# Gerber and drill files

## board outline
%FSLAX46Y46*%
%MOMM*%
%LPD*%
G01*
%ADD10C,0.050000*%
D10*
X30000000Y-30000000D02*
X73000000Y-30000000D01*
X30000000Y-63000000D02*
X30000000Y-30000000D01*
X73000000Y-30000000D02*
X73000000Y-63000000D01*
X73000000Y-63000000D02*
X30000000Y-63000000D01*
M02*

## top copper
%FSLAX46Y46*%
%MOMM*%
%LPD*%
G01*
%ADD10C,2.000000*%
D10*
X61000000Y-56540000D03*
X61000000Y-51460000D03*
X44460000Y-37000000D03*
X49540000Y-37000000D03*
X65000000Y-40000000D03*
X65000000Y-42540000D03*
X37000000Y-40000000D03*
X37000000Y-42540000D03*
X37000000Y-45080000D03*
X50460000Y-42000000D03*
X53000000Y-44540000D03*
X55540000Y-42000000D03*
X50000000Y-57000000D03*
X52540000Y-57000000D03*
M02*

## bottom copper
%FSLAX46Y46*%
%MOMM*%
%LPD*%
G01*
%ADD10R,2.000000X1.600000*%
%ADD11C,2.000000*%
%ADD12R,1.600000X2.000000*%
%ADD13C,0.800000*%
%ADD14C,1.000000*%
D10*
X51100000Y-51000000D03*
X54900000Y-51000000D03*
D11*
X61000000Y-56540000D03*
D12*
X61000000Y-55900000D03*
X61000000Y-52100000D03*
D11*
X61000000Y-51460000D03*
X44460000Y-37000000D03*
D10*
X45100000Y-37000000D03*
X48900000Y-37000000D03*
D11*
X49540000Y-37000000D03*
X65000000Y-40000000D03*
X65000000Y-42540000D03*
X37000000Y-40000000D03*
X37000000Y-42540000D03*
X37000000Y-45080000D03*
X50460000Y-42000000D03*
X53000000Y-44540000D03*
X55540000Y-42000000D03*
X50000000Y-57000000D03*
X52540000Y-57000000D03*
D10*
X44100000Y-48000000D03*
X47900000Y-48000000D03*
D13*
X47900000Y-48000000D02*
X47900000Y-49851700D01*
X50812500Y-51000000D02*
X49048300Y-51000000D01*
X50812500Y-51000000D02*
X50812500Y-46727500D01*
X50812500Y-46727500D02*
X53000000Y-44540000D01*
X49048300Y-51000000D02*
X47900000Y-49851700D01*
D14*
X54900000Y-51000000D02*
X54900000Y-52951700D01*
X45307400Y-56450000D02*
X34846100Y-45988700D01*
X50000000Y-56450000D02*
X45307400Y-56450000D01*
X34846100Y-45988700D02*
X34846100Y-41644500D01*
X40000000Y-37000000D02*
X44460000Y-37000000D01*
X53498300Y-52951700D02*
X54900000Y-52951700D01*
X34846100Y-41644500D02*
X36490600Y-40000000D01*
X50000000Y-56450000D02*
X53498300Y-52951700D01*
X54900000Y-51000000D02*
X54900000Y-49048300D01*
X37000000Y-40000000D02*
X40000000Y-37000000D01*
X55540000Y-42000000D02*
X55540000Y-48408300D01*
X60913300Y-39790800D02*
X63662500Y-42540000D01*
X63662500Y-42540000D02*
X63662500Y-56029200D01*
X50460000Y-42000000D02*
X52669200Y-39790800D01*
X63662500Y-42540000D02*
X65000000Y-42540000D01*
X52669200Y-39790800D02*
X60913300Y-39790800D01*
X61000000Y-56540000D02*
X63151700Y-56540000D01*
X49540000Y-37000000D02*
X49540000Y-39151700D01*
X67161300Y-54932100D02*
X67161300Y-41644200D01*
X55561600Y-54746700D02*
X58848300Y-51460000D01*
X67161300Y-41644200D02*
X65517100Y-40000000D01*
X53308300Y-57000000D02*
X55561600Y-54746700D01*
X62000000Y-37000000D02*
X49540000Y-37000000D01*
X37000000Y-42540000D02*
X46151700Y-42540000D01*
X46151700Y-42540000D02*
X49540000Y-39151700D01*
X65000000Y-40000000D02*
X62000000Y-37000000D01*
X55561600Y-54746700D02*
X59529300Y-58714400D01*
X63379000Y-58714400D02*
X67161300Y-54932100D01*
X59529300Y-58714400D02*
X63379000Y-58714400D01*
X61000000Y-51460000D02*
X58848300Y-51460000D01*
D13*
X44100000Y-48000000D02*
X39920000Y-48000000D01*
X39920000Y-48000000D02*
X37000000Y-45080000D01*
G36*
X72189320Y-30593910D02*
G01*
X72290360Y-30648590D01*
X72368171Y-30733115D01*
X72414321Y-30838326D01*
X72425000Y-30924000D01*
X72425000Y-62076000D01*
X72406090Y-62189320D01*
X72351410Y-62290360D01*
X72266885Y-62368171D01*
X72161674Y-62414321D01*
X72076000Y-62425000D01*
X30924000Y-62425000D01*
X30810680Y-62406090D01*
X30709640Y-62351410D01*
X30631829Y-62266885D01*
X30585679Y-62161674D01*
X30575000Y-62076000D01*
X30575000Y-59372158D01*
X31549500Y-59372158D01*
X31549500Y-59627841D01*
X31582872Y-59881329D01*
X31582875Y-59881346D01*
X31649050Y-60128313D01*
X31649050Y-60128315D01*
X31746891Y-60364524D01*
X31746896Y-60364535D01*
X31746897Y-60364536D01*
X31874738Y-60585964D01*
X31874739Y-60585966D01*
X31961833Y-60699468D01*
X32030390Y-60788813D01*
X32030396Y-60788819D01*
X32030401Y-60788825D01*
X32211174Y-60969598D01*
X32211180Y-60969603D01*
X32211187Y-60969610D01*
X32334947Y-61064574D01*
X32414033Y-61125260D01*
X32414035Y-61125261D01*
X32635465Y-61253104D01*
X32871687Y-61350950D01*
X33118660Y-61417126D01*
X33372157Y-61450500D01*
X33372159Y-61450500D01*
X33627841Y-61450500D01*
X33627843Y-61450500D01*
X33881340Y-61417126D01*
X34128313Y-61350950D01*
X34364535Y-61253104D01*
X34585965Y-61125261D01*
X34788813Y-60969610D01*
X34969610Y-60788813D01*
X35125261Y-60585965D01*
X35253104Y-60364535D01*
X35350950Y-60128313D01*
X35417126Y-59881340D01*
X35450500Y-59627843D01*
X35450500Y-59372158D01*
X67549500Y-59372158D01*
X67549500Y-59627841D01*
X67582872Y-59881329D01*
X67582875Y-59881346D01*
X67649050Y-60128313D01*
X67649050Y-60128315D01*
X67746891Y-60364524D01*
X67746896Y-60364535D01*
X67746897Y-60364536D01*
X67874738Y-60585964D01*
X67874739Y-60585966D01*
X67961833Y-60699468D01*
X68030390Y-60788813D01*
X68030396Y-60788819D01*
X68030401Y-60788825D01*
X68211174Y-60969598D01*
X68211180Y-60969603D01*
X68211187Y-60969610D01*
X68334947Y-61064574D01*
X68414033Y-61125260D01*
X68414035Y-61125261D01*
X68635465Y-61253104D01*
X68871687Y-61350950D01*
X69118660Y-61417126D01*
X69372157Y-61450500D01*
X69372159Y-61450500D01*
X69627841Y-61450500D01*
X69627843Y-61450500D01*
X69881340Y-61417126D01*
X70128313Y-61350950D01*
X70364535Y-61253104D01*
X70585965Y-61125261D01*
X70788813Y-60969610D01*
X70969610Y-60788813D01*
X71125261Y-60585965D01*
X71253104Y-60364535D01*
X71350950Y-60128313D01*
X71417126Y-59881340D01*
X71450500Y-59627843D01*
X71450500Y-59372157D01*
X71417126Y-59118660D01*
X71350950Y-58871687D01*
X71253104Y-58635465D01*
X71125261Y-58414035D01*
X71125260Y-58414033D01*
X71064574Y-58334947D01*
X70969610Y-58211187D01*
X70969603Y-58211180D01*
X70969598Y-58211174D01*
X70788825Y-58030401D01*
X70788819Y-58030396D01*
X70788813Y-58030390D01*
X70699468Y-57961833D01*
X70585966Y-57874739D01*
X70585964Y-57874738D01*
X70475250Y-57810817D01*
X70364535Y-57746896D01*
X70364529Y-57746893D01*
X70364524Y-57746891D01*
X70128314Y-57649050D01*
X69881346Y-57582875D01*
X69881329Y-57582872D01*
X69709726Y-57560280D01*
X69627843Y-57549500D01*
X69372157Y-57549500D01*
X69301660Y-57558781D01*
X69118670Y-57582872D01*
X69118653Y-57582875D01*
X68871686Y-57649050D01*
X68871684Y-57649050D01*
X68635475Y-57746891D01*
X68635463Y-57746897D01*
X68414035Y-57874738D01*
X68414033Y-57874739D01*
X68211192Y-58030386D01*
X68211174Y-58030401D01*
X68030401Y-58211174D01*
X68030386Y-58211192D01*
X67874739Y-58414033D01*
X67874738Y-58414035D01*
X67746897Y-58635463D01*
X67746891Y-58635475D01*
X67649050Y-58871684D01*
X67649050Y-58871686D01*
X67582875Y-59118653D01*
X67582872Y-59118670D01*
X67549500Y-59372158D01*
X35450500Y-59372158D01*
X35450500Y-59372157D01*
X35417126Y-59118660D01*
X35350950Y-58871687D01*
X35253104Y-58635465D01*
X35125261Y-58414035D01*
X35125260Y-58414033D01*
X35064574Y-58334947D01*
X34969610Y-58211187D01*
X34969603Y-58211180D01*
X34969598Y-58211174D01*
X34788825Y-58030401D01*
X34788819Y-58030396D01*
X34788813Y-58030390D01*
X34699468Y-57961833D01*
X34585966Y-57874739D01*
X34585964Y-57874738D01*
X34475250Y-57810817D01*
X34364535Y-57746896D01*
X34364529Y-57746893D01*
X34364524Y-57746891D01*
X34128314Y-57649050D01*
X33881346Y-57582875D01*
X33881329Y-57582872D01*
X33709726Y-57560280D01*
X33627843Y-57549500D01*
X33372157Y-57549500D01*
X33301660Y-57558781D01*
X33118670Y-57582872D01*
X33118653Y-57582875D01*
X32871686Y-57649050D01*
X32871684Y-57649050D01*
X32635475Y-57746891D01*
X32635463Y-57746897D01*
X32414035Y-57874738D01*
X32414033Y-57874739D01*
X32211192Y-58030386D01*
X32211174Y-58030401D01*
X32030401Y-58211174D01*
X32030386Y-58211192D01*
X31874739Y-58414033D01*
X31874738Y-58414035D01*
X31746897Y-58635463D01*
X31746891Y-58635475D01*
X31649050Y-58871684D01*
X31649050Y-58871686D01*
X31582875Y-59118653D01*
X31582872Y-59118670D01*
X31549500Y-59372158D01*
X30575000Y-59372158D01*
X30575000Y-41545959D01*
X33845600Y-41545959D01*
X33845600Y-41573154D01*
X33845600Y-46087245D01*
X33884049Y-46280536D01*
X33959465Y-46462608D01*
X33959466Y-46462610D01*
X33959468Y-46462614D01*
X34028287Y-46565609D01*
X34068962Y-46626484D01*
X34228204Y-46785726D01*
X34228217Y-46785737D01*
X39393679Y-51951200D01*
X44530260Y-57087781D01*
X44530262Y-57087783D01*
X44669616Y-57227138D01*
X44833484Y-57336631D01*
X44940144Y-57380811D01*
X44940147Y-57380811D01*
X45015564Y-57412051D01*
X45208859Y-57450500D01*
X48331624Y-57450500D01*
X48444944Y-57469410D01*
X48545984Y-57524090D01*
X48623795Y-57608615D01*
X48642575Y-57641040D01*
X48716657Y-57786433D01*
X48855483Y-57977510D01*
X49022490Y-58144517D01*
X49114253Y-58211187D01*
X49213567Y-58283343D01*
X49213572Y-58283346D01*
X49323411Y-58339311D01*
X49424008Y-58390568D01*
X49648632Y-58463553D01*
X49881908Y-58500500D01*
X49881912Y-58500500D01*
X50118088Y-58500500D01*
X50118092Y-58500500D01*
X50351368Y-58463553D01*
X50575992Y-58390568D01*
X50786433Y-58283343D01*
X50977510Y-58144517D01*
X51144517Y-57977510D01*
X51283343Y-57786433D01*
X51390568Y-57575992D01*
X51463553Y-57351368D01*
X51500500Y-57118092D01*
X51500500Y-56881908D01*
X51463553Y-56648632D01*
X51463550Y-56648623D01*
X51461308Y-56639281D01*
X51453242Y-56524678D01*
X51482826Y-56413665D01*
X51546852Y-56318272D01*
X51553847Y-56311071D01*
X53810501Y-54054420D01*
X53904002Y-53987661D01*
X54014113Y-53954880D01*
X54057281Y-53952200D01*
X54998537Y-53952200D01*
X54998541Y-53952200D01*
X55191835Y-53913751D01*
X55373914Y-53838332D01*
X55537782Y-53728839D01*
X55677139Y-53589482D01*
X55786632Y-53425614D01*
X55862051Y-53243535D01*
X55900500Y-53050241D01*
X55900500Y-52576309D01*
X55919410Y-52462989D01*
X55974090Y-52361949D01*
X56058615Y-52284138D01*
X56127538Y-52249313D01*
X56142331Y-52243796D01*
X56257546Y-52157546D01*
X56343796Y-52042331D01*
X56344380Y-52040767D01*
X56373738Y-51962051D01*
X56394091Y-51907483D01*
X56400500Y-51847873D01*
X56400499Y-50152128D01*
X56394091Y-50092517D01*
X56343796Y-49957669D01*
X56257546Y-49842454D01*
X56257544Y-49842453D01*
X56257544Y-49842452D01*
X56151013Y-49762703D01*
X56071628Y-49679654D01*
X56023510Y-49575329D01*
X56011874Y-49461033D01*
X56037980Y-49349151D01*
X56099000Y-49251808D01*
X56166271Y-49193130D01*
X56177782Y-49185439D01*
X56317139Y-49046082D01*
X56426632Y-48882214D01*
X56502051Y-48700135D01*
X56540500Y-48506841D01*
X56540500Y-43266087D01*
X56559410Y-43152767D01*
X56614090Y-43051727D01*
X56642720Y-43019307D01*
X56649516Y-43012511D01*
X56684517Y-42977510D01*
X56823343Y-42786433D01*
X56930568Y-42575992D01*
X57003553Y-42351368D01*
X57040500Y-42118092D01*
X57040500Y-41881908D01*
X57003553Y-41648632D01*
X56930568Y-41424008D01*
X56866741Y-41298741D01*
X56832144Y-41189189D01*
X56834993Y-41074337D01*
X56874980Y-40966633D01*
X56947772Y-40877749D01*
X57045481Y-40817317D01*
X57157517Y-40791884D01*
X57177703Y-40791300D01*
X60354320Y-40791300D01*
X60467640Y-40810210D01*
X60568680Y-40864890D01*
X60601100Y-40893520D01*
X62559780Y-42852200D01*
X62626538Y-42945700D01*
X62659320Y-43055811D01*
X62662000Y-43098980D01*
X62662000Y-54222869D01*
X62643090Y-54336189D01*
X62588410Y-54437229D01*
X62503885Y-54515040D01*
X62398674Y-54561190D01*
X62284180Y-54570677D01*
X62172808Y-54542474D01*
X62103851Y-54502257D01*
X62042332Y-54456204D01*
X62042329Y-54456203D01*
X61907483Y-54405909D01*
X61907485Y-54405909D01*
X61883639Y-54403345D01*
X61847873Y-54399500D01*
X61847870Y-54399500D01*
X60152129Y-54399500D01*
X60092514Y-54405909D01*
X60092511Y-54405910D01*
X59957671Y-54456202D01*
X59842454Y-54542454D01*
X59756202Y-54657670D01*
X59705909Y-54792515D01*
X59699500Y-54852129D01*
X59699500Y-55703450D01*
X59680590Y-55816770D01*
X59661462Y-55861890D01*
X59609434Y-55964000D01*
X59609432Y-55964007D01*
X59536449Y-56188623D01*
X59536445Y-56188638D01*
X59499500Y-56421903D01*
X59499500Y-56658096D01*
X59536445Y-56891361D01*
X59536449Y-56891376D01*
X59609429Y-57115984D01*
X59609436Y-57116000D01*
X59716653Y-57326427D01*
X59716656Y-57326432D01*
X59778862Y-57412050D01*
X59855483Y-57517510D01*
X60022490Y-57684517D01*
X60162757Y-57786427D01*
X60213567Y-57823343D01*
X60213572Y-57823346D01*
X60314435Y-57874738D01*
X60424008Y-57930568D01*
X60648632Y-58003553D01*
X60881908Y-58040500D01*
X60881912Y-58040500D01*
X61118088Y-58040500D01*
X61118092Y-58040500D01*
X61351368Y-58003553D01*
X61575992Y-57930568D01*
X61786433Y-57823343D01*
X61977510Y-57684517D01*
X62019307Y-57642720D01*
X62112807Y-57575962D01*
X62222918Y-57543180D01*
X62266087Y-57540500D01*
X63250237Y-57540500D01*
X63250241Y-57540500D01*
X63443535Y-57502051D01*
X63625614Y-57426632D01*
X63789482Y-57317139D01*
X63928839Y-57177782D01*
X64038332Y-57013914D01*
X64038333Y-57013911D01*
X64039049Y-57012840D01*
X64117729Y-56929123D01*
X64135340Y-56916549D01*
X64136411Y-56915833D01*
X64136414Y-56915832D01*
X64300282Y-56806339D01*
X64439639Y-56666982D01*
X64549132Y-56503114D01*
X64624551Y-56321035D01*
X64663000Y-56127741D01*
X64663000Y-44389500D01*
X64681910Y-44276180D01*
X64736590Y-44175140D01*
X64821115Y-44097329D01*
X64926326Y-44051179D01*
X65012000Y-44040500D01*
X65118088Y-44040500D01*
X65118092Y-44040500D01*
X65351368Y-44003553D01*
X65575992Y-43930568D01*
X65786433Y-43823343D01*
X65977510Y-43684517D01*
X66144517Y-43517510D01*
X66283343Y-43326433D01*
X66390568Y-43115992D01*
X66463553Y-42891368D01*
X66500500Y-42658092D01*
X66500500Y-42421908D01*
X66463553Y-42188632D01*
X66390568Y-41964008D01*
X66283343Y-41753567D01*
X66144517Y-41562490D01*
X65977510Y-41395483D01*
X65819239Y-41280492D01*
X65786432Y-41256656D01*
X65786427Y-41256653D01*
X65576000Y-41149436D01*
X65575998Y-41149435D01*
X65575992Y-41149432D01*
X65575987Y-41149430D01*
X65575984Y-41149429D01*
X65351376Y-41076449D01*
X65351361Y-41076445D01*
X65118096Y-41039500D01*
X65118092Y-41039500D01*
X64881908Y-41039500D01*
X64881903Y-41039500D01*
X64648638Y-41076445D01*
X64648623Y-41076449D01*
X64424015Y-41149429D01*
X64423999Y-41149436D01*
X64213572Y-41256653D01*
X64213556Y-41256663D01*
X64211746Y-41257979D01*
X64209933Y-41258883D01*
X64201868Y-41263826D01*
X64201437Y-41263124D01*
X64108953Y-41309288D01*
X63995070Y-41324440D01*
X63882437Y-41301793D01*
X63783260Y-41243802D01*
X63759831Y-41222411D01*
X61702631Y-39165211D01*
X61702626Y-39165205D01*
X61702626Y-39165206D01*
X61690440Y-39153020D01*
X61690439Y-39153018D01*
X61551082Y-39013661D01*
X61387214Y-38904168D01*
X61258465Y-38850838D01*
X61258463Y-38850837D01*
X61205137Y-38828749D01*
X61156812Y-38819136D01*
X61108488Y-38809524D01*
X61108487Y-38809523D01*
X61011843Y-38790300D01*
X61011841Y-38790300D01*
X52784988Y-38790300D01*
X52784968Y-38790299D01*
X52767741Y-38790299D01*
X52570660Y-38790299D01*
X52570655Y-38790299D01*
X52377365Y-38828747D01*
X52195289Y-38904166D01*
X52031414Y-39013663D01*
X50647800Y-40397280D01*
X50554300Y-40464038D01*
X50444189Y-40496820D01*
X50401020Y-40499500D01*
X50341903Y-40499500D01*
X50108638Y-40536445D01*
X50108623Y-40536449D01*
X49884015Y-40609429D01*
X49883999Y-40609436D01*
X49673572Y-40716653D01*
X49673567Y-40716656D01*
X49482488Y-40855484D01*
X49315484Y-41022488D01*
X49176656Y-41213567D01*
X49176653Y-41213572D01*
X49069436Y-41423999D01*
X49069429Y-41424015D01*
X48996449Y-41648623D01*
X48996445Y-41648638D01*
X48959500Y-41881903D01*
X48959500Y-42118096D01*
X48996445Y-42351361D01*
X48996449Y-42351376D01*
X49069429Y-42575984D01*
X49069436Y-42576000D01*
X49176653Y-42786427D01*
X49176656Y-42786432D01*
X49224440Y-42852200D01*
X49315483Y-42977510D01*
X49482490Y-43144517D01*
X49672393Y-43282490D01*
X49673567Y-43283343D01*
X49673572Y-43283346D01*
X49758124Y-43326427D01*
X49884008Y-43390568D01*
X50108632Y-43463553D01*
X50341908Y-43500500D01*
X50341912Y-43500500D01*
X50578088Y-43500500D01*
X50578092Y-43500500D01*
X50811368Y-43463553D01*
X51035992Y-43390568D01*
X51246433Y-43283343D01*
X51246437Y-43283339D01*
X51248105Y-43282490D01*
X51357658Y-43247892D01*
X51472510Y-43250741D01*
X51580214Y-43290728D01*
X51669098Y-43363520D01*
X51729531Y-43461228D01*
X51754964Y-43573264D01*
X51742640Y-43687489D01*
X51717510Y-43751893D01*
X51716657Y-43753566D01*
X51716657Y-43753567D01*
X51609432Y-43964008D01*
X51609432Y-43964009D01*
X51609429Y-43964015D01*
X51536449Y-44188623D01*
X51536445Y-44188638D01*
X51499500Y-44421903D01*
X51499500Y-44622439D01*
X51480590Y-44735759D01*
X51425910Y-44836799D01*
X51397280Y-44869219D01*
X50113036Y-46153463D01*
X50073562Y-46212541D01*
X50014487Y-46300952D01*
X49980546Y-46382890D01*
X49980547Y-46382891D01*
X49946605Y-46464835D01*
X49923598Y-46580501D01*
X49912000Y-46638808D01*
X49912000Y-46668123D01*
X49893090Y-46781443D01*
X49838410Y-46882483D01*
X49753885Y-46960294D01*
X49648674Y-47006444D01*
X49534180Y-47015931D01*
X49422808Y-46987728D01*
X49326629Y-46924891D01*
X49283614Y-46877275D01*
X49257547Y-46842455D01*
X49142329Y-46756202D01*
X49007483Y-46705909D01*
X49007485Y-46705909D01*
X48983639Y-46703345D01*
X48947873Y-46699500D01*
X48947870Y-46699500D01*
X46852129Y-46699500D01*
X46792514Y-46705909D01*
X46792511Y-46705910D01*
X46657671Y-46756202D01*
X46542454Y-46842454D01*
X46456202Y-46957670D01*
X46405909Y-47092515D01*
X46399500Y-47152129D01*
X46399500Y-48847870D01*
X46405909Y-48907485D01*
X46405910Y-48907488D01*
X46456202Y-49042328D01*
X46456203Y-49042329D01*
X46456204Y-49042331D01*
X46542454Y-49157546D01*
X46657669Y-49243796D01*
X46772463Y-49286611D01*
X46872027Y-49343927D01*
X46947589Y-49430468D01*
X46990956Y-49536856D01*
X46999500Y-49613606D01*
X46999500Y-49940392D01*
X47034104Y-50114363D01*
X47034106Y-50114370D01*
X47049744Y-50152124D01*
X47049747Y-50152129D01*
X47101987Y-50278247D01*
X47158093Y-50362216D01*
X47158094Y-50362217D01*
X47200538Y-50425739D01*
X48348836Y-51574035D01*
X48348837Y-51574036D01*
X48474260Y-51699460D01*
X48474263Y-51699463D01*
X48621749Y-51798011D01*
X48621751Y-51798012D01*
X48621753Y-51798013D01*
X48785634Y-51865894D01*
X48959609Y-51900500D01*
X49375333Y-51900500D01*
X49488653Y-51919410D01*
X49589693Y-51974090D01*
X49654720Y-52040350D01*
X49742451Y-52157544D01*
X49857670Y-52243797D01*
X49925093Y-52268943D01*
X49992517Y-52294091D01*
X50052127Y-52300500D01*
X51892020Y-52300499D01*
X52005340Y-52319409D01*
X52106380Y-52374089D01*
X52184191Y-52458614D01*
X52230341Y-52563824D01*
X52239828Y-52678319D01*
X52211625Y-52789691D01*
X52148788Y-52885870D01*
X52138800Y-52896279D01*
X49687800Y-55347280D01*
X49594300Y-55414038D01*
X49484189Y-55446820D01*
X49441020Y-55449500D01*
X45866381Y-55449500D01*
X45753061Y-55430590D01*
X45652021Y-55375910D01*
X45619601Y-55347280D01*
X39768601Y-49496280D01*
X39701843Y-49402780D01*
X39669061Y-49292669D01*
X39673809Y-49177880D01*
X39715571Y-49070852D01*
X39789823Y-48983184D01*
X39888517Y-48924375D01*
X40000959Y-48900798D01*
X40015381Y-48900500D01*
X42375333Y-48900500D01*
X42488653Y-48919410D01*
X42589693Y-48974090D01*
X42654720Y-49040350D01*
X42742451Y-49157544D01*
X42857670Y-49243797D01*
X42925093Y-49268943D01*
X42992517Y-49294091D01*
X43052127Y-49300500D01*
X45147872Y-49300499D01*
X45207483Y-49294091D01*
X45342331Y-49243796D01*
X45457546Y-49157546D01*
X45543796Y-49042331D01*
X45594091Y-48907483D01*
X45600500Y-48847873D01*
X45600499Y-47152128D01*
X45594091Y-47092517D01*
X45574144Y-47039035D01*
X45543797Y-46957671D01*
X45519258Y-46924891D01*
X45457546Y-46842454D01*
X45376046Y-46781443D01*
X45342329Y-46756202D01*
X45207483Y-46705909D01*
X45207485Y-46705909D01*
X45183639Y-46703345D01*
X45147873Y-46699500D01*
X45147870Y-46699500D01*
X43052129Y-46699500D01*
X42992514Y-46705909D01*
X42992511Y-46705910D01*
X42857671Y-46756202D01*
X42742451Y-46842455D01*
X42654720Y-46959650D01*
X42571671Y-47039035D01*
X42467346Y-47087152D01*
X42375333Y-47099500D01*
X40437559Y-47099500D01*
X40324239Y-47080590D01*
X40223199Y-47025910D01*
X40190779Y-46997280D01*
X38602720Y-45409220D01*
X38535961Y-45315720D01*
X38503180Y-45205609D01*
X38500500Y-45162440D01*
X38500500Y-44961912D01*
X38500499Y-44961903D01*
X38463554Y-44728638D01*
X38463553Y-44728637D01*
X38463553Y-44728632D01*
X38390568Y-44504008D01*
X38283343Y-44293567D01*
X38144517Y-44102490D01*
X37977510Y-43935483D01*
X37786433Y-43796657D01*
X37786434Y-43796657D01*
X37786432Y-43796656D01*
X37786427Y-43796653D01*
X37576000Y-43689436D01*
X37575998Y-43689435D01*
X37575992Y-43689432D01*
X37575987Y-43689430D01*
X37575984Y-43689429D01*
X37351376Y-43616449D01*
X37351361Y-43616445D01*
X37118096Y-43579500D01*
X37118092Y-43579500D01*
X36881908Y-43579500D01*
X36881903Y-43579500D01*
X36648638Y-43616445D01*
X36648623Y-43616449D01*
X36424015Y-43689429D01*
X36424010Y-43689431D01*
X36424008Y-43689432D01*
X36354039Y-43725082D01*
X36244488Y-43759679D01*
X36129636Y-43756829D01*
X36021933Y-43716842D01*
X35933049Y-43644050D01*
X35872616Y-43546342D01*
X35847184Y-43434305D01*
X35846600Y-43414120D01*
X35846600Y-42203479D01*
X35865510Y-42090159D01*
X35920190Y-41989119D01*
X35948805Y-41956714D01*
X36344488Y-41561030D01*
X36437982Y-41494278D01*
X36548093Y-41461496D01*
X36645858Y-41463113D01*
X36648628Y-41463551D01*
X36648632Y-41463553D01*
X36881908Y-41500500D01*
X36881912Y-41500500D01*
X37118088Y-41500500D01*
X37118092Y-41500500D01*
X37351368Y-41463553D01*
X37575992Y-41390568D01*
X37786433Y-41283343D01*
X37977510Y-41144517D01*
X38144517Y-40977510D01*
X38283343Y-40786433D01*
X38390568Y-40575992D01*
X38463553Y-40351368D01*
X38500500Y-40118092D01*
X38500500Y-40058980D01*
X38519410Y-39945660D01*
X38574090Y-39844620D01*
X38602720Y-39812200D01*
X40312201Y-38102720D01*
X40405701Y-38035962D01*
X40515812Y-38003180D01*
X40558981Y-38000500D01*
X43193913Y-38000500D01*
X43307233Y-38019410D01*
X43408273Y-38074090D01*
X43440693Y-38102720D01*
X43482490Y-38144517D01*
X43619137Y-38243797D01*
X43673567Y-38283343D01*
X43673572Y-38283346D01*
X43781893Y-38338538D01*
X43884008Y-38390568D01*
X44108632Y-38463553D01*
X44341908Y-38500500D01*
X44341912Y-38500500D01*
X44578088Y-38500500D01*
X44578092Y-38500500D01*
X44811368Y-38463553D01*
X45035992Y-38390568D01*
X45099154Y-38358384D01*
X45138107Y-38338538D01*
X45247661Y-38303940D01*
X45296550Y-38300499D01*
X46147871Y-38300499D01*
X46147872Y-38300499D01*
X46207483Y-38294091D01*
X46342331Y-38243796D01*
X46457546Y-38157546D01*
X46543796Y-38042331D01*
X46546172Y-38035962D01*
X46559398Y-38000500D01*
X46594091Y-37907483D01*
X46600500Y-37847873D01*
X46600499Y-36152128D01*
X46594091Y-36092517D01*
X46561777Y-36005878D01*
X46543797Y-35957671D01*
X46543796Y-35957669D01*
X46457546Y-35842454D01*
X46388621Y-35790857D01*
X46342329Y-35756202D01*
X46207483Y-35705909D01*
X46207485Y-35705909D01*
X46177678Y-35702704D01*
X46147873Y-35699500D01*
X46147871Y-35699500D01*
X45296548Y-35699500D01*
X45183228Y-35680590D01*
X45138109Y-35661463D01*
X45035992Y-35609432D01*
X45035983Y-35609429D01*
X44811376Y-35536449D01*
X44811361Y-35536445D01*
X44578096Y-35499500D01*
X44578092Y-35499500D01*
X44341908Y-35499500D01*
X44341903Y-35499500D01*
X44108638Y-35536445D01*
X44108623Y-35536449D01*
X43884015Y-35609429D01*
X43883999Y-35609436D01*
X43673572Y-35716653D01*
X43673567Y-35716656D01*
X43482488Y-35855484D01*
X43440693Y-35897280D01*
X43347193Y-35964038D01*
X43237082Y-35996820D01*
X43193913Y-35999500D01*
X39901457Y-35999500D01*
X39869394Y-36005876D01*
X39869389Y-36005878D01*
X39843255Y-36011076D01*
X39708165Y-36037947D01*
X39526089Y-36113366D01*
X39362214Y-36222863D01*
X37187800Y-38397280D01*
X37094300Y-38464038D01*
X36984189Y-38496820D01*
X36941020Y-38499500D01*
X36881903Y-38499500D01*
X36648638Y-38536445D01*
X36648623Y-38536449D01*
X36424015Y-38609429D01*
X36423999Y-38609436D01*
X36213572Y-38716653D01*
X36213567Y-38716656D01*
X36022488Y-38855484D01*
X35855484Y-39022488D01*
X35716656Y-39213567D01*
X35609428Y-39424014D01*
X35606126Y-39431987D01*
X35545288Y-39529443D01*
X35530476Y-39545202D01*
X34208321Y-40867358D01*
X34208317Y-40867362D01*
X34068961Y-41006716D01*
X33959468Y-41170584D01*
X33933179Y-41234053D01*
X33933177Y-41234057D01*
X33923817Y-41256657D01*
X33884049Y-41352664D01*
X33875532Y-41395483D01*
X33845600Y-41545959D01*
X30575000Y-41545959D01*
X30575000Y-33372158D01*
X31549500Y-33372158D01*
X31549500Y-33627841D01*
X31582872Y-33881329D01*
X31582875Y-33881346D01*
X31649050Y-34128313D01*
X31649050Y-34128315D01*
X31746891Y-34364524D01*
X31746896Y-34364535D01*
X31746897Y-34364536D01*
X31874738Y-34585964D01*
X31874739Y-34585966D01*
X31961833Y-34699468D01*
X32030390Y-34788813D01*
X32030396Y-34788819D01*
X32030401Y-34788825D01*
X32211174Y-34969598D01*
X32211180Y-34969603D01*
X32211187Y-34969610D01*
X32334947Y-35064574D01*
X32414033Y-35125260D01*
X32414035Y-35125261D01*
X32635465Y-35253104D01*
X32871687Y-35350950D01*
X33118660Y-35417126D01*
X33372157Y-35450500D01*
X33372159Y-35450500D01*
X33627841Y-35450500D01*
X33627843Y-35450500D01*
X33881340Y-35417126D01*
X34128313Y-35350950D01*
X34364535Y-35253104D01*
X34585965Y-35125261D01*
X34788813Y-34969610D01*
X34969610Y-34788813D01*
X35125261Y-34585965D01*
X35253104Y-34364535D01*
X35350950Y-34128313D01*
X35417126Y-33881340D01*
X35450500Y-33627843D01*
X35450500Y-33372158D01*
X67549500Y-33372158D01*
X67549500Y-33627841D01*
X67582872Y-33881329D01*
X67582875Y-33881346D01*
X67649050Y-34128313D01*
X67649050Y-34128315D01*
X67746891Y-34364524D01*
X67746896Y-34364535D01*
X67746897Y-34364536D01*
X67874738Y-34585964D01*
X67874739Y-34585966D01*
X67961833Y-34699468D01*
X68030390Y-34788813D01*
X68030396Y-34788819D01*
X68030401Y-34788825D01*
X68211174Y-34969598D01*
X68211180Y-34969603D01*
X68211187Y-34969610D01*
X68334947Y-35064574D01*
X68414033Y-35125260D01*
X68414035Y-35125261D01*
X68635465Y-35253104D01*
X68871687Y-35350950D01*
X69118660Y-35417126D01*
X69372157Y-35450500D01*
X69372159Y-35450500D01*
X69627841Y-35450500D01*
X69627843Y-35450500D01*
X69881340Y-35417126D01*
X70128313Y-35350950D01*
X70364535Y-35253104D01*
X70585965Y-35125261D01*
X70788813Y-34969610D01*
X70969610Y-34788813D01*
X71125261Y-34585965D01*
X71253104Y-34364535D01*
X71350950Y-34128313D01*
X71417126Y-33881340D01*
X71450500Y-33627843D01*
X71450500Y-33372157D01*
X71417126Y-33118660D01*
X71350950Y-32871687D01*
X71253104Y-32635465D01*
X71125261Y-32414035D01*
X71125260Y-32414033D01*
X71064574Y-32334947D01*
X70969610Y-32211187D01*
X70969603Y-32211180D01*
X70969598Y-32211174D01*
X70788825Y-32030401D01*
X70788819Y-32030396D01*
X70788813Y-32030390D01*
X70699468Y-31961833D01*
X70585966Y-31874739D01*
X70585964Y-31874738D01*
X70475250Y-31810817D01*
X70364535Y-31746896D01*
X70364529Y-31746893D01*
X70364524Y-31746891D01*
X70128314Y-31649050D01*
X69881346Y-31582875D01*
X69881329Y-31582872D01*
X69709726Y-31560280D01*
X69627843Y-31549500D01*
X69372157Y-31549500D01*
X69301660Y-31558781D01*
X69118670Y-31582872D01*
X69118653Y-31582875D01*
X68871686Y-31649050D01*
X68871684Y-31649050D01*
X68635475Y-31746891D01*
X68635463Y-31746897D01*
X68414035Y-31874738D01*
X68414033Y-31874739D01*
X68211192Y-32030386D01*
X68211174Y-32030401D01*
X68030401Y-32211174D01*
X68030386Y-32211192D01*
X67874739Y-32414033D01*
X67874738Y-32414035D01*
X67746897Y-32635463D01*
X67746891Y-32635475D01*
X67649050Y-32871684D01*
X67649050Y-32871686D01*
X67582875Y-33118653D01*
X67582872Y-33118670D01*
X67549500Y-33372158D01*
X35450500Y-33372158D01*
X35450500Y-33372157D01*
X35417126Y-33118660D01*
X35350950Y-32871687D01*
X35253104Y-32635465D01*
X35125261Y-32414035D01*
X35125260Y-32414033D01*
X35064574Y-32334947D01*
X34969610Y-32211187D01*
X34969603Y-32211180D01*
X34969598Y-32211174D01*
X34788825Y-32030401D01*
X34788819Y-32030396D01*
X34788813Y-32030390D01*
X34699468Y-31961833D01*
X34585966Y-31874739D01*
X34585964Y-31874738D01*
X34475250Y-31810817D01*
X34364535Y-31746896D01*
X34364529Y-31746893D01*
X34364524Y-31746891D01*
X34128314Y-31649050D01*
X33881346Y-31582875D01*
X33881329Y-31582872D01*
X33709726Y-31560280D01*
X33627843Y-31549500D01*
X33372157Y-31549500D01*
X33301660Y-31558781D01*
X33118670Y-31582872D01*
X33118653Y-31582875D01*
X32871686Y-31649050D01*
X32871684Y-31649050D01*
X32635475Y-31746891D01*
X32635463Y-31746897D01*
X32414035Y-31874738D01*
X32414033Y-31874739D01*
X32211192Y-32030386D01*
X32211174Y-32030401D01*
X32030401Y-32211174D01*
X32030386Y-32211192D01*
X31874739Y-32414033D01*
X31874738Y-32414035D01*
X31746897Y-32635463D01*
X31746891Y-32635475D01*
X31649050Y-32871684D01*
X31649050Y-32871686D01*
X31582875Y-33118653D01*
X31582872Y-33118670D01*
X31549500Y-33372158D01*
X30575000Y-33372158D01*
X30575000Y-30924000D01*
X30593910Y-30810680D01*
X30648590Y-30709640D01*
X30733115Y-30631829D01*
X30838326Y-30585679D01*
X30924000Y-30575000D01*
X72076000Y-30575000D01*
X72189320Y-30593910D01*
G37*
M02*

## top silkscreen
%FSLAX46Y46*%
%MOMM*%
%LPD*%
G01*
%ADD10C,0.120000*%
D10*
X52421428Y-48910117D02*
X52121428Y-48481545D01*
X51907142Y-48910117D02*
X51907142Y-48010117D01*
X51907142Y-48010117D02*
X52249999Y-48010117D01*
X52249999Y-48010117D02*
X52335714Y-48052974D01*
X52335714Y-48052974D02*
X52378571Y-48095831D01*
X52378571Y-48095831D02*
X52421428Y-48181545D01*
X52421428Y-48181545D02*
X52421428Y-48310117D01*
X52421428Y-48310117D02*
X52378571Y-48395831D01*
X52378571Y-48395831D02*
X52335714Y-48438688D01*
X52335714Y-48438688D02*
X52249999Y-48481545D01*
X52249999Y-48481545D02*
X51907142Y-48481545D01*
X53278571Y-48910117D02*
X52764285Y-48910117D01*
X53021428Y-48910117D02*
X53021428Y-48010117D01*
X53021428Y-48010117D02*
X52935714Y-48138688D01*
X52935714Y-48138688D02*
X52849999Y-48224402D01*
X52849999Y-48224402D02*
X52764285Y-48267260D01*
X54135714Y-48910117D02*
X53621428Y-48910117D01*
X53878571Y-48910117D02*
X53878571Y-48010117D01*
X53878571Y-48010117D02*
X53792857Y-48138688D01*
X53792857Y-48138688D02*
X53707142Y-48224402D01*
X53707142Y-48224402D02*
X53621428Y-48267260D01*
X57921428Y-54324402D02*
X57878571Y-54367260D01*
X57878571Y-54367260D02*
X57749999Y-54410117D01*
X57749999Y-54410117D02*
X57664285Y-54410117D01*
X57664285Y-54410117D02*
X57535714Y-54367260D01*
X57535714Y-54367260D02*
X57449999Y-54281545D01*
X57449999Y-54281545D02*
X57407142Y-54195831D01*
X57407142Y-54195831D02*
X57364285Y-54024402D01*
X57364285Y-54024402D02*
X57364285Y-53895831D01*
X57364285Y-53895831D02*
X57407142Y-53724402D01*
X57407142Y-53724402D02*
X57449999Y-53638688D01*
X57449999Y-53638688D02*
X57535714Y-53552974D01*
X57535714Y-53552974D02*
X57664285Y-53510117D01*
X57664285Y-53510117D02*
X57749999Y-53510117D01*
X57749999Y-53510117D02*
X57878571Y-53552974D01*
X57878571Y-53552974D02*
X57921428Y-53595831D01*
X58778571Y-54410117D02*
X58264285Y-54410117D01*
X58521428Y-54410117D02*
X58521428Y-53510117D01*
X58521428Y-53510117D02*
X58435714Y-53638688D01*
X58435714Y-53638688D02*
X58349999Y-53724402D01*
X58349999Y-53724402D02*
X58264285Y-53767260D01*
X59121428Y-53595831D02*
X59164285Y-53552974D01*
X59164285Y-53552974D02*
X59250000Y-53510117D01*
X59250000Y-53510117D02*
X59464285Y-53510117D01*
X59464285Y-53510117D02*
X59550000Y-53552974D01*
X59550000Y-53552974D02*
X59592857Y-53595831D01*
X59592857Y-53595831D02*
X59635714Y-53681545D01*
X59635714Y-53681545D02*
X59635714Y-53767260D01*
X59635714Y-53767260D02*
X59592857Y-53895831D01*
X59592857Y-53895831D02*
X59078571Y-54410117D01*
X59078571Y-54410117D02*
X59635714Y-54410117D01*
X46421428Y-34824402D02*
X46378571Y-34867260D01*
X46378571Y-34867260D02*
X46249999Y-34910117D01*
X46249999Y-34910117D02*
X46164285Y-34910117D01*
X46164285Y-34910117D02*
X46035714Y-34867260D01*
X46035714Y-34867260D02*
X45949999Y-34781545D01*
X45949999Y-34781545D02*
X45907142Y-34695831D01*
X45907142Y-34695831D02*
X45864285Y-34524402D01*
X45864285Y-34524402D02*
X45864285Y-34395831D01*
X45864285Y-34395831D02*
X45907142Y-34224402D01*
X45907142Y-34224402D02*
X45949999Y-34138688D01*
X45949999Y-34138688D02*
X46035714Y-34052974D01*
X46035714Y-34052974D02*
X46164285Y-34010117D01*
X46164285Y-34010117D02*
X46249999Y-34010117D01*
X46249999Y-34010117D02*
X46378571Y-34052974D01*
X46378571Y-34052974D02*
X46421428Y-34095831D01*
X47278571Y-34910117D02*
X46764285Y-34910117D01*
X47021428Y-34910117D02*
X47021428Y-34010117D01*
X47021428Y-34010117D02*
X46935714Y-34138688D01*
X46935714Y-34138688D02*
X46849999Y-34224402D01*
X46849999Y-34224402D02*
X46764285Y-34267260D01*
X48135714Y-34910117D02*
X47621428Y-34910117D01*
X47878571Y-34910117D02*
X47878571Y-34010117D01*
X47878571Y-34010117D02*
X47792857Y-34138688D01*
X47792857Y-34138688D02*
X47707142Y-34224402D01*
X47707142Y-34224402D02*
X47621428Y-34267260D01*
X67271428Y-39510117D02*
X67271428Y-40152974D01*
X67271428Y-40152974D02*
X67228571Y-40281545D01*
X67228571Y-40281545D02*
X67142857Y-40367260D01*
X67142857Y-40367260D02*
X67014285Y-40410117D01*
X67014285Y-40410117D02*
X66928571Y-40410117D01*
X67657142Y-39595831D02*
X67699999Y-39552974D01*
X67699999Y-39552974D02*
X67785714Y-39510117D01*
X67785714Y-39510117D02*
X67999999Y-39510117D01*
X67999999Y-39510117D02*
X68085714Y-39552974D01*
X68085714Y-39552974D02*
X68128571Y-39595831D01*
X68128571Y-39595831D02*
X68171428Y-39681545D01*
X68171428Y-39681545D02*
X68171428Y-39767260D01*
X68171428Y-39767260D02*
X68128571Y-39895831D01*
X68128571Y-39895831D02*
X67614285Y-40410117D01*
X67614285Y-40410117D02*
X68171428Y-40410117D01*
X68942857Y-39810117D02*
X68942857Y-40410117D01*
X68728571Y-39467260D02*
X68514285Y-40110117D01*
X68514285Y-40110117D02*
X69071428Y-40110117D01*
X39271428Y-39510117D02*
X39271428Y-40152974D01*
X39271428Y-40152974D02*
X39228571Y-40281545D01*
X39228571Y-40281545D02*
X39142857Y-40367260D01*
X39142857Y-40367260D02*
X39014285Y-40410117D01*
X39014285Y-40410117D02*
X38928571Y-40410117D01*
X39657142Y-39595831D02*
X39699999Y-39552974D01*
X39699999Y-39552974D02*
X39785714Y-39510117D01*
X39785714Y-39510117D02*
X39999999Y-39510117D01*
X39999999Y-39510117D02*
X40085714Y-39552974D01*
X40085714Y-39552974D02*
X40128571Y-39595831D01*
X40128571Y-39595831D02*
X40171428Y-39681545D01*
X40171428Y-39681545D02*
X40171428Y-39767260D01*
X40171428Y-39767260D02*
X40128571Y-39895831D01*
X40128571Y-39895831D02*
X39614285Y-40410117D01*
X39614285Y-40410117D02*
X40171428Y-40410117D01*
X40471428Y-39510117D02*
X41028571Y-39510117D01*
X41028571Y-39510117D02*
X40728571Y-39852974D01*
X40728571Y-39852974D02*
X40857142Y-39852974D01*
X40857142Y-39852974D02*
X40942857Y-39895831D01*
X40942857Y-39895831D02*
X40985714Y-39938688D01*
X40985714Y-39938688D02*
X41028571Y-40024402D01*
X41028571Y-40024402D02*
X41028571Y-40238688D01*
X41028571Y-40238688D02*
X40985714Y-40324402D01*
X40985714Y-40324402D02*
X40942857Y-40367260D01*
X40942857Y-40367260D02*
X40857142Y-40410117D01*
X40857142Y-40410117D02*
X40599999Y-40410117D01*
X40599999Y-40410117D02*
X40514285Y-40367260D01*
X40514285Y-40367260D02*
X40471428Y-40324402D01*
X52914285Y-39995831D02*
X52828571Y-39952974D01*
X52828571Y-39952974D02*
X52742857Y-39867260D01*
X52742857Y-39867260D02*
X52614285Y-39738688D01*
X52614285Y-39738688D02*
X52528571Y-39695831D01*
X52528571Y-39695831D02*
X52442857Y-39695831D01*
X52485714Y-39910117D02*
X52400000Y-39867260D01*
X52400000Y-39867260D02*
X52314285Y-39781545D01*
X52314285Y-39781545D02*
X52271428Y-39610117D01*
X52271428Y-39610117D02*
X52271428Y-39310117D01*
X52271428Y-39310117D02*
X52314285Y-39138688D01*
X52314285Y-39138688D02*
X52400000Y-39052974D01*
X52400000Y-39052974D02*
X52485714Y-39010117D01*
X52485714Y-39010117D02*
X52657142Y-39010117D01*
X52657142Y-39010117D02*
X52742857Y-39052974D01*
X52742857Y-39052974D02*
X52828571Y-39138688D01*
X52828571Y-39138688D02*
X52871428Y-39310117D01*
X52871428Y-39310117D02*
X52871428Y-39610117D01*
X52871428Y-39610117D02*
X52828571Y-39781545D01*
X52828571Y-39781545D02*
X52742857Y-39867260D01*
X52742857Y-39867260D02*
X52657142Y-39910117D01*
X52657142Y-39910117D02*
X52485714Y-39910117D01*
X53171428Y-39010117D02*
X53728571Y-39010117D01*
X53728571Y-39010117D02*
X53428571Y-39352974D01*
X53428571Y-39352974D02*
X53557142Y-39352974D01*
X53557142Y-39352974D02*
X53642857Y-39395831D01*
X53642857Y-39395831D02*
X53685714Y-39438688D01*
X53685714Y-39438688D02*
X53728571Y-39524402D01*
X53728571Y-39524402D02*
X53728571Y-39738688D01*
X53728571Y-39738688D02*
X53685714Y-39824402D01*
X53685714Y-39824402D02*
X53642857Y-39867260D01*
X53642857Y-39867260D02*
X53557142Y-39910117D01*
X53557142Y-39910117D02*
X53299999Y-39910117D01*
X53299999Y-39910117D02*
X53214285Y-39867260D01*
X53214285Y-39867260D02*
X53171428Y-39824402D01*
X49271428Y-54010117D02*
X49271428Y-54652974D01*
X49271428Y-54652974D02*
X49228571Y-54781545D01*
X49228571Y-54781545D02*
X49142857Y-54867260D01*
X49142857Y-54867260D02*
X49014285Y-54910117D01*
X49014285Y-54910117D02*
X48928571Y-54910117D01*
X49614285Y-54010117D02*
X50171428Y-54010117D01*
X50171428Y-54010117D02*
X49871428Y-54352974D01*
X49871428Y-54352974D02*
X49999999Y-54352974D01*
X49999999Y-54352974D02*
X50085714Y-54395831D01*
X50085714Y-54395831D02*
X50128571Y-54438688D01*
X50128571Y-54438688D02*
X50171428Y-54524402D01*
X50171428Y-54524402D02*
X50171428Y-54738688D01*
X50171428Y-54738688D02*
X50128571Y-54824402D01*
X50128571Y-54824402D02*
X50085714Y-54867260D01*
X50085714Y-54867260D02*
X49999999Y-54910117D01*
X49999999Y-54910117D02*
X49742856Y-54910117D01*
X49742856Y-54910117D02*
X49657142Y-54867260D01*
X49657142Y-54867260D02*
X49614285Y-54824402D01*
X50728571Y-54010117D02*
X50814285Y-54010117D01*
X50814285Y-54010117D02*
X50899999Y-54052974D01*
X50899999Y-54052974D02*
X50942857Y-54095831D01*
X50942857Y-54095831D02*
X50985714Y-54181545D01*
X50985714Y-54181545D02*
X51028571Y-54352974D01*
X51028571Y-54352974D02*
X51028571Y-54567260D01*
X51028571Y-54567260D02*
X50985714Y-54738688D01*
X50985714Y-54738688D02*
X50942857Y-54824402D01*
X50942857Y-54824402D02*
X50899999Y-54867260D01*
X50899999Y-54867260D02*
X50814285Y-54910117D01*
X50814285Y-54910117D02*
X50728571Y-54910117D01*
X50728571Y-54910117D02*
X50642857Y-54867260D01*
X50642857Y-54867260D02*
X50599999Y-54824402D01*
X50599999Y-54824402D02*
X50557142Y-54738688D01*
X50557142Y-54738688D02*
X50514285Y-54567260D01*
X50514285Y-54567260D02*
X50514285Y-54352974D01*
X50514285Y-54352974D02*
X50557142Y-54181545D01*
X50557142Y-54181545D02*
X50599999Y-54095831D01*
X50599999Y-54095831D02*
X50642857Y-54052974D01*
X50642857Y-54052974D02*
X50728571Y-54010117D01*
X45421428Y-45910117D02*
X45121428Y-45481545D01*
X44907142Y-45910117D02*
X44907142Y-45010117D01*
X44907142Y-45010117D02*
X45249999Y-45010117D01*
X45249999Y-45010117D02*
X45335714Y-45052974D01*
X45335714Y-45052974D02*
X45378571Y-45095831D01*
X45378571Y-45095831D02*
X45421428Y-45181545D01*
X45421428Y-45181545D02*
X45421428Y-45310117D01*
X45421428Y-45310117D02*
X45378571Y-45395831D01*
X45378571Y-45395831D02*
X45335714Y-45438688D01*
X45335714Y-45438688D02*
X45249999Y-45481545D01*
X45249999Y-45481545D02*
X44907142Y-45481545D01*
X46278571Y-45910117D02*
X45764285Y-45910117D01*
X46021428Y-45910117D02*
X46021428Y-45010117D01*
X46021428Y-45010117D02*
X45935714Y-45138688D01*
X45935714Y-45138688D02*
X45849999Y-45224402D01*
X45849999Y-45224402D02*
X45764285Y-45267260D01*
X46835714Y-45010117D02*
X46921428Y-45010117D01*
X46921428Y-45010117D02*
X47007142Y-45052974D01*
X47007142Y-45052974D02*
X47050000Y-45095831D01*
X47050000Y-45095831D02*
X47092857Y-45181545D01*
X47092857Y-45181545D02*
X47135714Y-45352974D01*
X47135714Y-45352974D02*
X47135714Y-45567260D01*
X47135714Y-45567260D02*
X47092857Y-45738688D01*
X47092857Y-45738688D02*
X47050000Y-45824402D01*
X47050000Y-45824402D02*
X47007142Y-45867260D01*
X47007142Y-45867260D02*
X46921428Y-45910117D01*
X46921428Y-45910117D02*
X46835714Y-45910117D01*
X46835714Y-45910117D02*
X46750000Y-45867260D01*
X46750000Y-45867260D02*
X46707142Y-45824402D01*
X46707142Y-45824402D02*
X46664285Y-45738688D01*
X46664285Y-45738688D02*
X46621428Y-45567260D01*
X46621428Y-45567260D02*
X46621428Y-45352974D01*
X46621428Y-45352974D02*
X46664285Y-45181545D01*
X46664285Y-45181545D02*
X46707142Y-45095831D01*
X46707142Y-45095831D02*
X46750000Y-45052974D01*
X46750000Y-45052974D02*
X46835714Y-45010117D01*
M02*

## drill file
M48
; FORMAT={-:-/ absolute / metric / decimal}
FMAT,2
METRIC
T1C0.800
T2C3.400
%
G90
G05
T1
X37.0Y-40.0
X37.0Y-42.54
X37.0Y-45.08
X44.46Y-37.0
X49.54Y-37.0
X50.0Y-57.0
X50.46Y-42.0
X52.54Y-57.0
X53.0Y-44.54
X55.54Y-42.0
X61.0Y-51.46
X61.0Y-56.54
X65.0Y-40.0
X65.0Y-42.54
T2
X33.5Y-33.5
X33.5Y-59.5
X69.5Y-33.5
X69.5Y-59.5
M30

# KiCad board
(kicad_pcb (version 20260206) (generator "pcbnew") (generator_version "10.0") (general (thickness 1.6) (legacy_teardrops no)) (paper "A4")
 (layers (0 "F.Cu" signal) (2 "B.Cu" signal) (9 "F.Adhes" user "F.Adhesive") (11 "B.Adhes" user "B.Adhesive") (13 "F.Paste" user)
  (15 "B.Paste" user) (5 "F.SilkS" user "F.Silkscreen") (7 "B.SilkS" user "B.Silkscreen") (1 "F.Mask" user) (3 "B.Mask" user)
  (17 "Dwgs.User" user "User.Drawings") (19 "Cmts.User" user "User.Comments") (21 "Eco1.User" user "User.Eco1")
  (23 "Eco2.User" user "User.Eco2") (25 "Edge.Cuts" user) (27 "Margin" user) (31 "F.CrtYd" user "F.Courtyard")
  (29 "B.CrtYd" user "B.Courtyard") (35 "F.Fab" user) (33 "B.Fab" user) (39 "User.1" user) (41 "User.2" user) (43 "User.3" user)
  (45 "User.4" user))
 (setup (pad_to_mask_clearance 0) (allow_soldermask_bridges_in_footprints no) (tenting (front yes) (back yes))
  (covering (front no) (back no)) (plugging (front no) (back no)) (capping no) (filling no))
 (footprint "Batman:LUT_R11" (layer "F.Cu") (at 53 51)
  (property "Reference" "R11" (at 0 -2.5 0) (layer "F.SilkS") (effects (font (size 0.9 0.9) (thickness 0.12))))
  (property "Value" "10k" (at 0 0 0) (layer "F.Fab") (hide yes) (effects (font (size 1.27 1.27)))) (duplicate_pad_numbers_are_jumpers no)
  (pad "1" smd rect (at -1.9 0) (size 2 1.6) (layers "B.Cu") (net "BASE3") (thermal_bridge_angle 45))
  (pad "2" smd rect (at 1.9 0) (size 2 1.6) (layers "B.Cu") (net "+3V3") (thermal_bridge_angle 45)))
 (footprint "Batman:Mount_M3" (layer "F.Cu") (at 69.5 33.5)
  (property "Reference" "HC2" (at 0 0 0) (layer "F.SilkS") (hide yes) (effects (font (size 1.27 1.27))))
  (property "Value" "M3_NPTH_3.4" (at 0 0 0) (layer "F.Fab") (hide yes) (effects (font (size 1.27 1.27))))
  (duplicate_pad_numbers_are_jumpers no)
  (pad "" np_thru_hole circle (at 0 0) (size 3.4 3.4) (drill 3.4) (layers "*.Cu")))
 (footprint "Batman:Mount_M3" (layer "F.Cu") (at 33.5 59.5)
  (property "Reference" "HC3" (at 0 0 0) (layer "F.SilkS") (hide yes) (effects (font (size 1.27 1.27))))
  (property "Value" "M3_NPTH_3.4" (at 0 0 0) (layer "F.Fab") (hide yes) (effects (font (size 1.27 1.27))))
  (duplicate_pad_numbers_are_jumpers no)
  (pad "" np_thru_hole circle (at 0 0) (size 3.4 3.4) (drill 3.4) (layers "*.Cu")))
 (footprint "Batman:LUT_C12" (layer "F.Cu") (at 61 54 90)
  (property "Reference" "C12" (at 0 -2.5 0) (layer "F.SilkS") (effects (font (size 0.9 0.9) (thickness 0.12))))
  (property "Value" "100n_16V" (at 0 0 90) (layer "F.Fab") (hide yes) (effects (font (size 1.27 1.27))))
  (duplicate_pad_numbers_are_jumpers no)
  (pad "1" thru_hole circle (at -2.54 0 90) (size 2 2) (drill 0.8) (layers "*.Cu") (remove_unused_layers no) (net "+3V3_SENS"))
  (pad "1" smd rect (at -1.9 0 90) (size 2 1.6) (layers "B.Cu") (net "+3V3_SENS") (thermal_bridge_angle 45))
  (pad "2" smd rect (at 1.9 0 90) (size 2 1.6) (layers "B.Cu") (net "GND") (thermal_bridge_angle 45))
  (pad "2" thru_hole circle (at 2.54 0 90) (size 2 2) (drill 0.8) (layers "*.Cu") (remove_unused_layers no) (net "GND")))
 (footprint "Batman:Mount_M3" (layer "F.Cu") (at 33.5 33.5)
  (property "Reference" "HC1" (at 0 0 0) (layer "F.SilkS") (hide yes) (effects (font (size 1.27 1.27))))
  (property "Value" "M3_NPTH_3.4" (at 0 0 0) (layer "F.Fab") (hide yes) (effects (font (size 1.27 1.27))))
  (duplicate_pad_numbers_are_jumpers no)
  (pad "" np_thru_hole circle (at 0 0) (size 3.4 3.4) (drill 3.4) (layers "*.Cu")))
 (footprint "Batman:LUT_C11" (layer "F.Cu") (at 47 37)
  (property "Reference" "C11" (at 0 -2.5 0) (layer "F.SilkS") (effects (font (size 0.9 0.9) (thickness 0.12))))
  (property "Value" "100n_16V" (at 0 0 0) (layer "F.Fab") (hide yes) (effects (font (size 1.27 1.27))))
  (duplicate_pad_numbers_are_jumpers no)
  (pad "1" thru_hole circle (at -2.54 0) (size 2 2) (drill 0.8) (layers "*.Cu") (remove_unused_layers no) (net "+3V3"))
  (pad "1" smd rect (at -1.9 0) (size 2 1.6) (layers "B.Cu") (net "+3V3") (thermal_bridge_angle 45))
  (pad "2" smd rect (at 1.9 0) (size 2 1.6) (layers "B.Cu") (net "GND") (thermal_bridge_angle 45))
  (pad "2" thru_hole circle (at 2.54 0) (size 2 2) (drill 0.8) (layers "*.Cu") (remove_unused_layers no) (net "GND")))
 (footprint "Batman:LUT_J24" (layer "F.Cu") (at 65 40 -90)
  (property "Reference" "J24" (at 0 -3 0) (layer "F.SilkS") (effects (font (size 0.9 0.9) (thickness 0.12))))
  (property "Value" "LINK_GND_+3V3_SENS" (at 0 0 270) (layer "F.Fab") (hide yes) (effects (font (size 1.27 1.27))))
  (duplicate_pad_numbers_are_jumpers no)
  (pad "1" thru_hole circle (at 0 0 270) (size 2 2) (drill 0.8) (layers "*.Cu") (remove_unused_layers no) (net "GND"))
  (pad "2" thru_hole circle (at 2.54 0 270) (size 2 2) (drill 0.8) (layers "*.Cu") (remove_unused_layers no) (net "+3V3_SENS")))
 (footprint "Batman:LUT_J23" (layer "F.Cu") (at 37 40 -90)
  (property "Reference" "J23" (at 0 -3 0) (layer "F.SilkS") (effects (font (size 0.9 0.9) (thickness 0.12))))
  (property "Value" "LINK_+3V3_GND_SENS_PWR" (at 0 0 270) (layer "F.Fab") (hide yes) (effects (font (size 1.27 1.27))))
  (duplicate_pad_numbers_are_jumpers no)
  (pad "1" thru_hole circle (at 0 0 270) (size 2 2) (drill 0.8) (layers "*.Cu") (remove_unused_layers no) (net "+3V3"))
  (pad "2" thru_hole circle (at 2.54 0 270) (size 2 2) (drill 0.8) (layers "*.Cu") (remove_unused_layers no) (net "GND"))
  (pad "3" thru_hole circle (at 5.08 0 270) (size 2 2) (drill 0.8) (layers "*.Cu") (remove_unused_layers no) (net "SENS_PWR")))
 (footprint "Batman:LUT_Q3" (layer "F.Cu") (at 53 42)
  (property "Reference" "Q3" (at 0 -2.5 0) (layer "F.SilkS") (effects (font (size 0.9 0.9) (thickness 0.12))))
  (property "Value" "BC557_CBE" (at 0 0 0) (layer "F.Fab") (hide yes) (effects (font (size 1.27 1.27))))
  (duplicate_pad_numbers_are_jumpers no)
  (pad "1" thru_hole circle (at -2.54 0) (size 2 2) (drill 0.8) (layers "*.Cu") (remove_unused_layers no) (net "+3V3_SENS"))
  (pad "2" thru_hole circle (at 0 2.54) (size 2 2) (drill 0.8) (layers "*.Cu") (remove_unused_layers no) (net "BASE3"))
  (pad "3" thru_hole circle (at 2.54 0) (size 2 2) (drill 0.8) (layers "*.Cu") (remove_unused_layers no) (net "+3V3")))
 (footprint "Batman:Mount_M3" (layer "F.Cu") (at 69.5 59.5)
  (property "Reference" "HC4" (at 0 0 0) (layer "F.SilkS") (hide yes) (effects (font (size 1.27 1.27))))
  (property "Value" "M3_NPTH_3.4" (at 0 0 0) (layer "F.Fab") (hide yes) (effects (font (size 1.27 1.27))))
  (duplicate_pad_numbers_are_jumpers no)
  (pad "" np_thru_hole circle (at 0 0) (size 3.4 3.4) (drill 3.4) (layers "*.Cu")))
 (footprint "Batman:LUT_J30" (layer "F.Cu") (at 50 57)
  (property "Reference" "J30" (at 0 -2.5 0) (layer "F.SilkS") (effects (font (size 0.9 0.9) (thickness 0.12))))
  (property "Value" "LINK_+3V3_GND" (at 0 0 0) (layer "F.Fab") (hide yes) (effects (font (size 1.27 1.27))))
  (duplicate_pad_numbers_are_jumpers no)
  (pad "1" thru_hole circle (at 0 0) (size 2 2) (drill 0.8) (layers "*.Cu") (remove_unused_layers no) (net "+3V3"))
  (pad "2" thru_hole circle (at 2.54 0) (size 2 2) (drill 0.8) (layers "*.Cu") (remove_unused_layers no) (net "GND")))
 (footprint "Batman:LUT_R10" (layer "F.Cu") (at 46 48)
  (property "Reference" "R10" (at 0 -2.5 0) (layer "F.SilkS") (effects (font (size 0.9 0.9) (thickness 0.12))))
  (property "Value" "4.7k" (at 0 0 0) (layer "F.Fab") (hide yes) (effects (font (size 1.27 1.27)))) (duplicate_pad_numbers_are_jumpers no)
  (pad "1" smd rect (at -1.9 0) (size 2 1.6) (layers "B.Cu") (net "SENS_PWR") (thermal_bridge_angle 45))
  (pad "2" smd rect (at 1.9 0) (size 2 1.6) (layers "B.Cu") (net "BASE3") (thermal_bridge_angle 45)))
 (gr_line (start 30 30) (end 73 30) (stroke (width 0.05) (type default)) (layer "Edge.Cuts"))
 (gr_line (start 30 63) (end 30 30) (stroke (width 0.05) (type default)) (layer "Edge.Cuts"))
 (gr_line (start 73 30) (end 73 63) (stroke (width 0.05) (type default)) (layer "Edge.Cuts"))
 (gr_line (start 73 63) (end 30 63) (stroke (width 0.05) (type default)) (layer "Edge.Cuts"))
 (segment (start 47.9 48) (end 47.9 49.8517) (width 0.8) (layer "B.Cu") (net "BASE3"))
 (segment (start 50.8125 51) (end 49.0483 51) (width 0.8) (layer "B.Cu") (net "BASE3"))
 (segment (start 50.8125 51) (end 50.8125 46.7275) (width 0.8) (layer "B.Cu") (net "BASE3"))
 (segment (start 50.8125 46.7275) (end 53 44.54) (width 0.8) (layer "B.Cu") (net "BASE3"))
 (segment (start 49.0483 51) (end 47.9 49.8517) (width 0.8) (layer "B.Cu") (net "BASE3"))
 (segment (start 54.9 51) (end 54.9 52.9517) (width 1) (layer "B.Cu") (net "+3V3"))
 (segment (start 45.3074 56.45) (end 34.8461 45.9887) (width 1) (layer "B.Cu") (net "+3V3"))
 (segment (start 50 56.45) (end 45.3074 56.45) (width 1) (layer "B.Cu") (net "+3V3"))
 (segment (start 34.8461 45.9887) (end 34.8461 41.6445) (width 1) (layer "B.Cu") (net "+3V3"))
 (segment (start 40 37) (end 44.46 37) (width 1) (layer "B.Cu") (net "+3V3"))
 (segment (start 53.4983 52.9517) (end 54.9 52.9517) (width 1) (layer "B.Cu") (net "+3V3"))
 (segment (start 34.8461 41.6445) (end 36.4906 40) (width 1) (layer "B.Cu") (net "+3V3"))
 (segment (start 50 56.45) (end 53.4983 52.9517) (width 1) (layer "B.Cu") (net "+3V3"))
 (segment (start 54.9 51) (end 54.9 49.0483) (width 1) (layer "B.Cu") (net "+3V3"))
 (segment (start 37 40) (end 40 37) (width 1) (layer "B.Cu") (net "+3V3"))
 (segment (start 55.54 42) (end 55.54 48.4083) (width 1) (layer "B.Cu") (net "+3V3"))
 (segment (start 60.9133 39.7908) (end 63.6625 42.54) (width 1) (layer "B.Cu") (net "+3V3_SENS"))
 (segment (start 63.6625 42.54) (end 63.6625 56.0292) (width 1) (layer "B.Cu") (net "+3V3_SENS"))
 (segment (start 50.46 42) (end 52.6692 39.7908) (width 1) (layer "B.Cu") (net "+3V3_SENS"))
 (segment (start 63.6625 42.54) (end 65 42.54) (width 1) (layer "B.Cu") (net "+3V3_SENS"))
 (segment (start 52.6692 39.7908) (end 60.9133 39.7908) (width 1) (layer "B.Cu") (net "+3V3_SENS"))
 (segment (start 61 56.54) (end 63.1517 56.54) (width 1) (layer "B.Cu") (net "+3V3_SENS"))
 (segment (start 49.54 37) (end 49.54 39.1517) (width 1) (layer "B.Cu") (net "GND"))
 (segment (start 67.1613 54.9321) (end 67.1613 41.6442) (width 1) (layer "B.Cu") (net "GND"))
 (segment (start 55.5616 54.7467) (end 58.8483 51.46) (width 1) (layer "B.Cu") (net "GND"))
 (segment (start 67.1613 41.6442) (end 65.5171 40) (width 1) (layer "B.Cu") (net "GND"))
 (segment (start 53.3083 57) (end 55.5616 54.7467) (width 1) (layer "B.Cu") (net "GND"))
 (segment (start 62 37) (end 49.54 37) (width 1) (layer "B.Cu") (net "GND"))
 (segment (start 37 42.54) (end 46.1517 42.54) (width 1) (layer "B.Cu") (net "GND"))
 (segment (start 46.1517 42.54) (end 49.54 39.1517) (width 1) (layer "B.Cu") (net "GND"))
 (segment (start 65 40) (end 62 37) (width 1) (layer "B.Cu") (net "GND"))
 (segment (start 55.5616 54.7467) (end 59.5293 58.7144) (width 1) (layer "B.Cu") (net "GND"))
 (segment (start 63.379 58.7144) (end 67.1613 54.9321) (width 1) (layer "B.Cu") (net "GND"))
 (segment (start 59.5293 58.7144) (end 63.379 58.7144) (width 1) (layer "B.Cu") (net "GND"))
 (segment (start 61 51.46) (end 58.8483 51.46) (width 1) (layer "B.Cu") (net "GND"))
 (segment (start 44.1 48) (end 39.92 48) (width 0.8) (layer "B.Cu") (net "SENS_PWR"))
 (segment (start 39.92 48) (end 37 45.08) (width 0.8) (layer "B.Cu") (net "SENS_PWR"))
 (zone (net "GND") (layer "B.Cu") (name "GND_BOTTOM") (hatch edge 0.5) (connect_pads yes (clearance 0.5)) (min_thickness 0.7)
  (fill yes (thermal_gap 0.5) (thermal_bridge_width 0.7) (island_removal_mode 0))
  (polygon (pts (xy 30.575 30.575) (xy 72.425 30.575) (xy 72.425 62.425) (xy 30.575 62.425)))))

